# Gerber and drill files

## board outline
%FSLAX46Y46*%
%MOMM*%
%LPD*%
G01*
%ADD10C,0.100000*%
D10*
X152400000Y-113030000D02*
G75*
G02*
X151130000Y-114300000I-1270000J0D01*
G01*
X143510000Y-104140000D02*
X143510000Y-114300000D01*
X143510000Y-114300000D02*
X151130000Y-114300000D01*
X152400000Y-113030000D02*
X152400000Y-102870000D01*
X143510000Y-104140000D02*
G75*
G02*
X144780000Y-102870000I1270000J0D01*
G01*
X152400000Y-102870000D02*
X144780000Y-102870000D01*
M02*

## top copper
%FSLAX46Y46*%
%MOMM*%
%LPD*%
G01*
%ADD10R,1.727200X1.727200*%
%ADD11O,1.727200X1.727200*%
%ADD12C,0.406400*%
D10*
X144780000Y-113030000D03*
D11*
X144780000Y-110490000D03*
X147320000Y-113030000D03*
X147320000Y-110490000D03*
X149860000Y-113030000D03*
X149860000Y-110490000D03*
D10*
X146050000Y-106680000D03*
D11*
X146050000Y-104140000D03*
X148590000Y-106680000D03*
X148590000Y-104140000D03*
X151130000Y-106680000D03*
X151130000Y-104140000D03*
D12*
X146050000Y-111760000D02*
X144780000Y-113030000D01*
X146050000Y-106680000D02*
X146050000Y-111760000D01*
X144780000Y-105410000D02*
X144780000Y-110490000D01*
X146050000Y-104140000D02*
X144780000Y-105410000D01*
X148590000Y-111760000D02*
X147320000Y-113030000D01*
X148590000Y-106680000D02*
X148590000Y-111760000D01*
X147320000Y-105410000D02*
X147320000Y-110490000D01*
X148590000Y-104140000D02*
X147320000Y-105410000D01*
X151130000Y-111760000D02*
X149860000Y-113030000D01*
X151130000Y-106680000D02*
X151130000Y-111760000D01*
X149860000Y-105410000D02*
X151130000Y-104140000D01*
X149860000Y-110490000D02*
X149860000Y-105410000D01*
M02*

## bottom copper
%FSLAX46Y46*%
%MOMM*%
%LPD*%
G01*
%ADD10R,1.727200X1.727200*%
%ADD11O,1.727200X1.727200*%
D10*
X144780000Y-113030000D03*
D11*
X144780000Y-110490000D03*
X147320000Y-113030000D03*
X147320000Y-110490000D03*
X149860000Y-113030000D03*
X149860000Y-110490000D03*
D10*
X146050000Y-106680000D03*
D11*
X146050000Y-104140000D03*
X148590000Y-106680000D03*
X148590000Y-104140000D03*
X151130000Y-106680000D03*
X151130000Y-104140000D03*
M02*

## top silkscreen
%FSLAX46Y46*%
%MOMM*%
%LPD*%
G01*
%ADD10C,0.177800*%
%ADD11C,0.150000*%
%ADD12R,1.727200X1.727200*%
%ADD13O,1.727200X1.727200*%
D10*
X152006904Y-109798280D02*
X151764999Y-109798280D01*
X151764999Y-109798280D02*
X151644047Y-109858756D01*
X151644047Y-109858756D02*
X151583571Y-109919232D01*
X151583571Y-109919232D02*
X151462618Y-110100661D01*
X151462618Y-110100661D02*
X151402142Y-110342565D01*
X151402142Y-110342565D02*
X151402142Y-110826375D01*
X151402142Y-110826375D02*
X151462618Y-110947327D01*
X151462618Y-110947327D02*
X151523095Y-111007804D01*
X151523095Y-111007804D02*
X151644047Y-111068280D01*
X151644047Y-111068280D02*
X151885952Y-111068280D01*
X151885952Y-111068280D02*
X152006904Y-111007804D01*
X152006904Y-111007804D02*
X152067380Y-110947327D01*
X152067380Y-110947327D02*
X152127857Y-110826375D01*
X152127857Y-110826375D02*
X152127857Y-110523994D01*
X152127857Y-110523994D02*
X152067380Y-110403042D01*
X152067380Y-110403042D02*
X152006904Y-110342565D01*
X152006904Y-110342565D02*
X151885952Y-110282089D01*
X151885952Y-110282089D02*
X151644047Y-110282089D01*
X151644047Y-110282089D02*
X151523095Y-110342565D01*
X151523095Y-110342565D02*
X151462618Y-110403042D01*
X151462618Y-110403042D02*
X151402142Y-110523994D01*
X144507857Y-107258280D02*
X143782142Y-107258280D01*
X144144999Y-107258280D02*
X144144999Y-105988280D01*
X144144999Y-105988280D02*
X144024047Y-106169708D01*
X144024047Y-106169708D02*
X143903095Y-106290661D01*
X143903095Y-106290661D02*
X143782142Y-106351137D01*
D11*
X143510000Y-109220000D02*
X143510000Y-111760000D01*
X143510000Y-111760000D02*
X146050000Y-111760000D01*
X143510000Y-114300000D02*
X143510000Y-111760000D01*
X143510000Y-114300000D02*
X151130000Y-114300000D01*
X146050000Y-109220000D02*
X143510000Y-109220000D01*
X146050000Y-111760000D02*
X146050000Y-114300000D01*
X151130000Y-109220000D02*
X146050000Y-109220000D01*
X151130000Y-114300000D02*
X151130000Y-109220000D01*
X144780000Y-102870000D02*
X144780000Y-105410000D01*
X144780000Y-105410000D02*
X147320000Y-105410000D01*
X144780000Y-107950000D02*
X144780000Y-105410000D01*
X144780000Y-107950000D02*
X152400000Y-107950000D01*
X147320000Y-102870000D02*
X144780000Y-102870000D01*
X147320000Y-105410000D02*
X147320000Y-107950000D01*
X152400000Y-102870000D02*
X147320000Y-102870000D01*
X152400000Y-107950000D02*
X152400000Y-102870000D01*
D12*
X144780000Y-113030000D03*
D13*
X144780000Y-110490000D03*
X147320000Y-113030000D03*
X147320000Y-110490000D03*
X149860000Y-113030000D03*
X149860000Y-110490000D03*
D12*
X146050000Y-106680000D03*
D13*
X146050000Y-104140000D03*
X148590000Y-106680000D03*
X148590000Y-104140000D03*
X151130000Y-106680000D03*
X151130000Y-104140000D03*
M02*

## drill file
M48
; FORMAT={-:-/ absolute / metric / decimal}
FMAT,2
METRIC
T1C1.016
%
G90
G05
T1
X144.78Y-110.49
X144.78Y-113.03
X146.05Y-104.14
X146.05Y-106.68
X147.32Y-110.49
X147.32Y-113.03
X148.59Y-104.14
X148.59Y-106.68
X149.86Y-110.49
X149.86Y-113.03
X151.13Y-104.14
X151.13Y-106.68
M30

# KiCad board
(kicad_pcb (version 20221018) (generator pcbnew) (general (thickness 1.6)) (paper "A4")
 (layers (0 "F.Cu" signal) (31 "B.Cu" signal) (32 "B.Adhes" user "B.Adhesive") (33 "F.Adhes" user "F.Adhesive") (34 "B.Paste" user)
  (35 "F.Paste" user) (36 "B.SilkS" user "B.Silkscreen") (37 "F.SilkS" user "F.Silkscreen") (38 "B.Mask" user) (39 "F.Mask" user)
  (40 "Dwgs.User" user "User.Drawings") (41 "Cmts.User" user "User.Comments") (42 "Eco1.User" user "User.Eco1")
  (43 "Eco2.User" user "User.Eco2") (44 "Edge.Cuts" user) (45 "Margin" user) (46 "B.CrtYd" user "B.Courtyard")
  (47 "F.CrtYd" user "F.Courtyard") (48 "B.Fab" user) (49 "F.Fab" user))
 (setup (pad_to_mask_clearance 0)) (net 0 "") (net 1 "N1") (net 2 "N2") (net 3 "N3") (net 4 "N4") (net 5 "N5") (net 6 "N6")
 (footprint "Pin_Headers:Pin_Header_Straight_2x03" (layer "F.Cu") (at 147.32 111.76)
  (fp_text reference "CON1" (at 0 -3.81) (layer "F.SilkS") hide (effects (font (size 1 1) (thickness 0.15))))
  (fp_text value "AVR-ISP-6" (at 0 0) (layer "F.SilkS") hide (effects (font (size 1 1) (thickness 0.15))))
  (fp_line (start -3.81 -2.54) (end -3.81 0) (stroke (width 0.15) (type solid)) (layer "F.SilkS"))
  (fp_line (start -3.81 0) (end -1.27 0) (stroke (width 0.15) (type solid)) (layer "F.SilkS"))
  (fp_line (start -3.81 2.54) (end -3.81 0) (stroke (width 0.15) (type solid)) (layer "F.SilkS"))
  (fp_line (start -3.81 2.54) (end 3.81 2.54) (stroke (width 0.15) (type solid)) (layer "F.SilkS"))
  (fp_line (start -1.27 -2.54) (end -3.81 -2.54) (stroke (width 0.15) (type solid)) (layer "F.SilkS"))
  (fp_line (start -1.27 0) (end -1.27 2.54) (stroke (width 0.15) (type solid)) (layer "F.SilkS"))
  (fp_line (start 3.81 -2.54) (end -1.27 -2.54) (stroke (width 0.15) (type solid)) (layer "F.SilkS"))
  (fp_line (start 3.81 2.54) (end 3.81 -2.54) (stroke (width 0.15) (type solid)) (layer "F.SilkS"))
  (pad "1" thru_hole rect (at -2.54 1.27) (size 1.7272 1.7272) (drill 1.016) (layers "*.Cu" "*.Mask" "F.SilkS") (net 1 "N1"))
  (pad "2" thru_hole oval (at -2.54 -1.27) (size 1.7272 1.7272) (drill 1.016) (layers "*.Cu" "*.Mask" "F.SilkS") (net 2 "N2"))
  (pad "3" thru_hole oval (at 0 1.27) (size 1.7272 1.7272) (drill 1.016) (layers "*.Cu" "*.Mask" "F.SilkS") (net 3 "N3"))
  (pad "4" thru_hole oval (at 0 -1.27) (size 1.7272 1.7272) (drill 1.016) (layers "*.Cu" "*.Mask" "F.SilkS") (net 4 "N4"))
  (pad "5" thru_hole oval (at 2.54 1.27) (size 1.7272 1.7272) (drill 1.016) (layers "*.Cu" "*.Mask" "F.SilkS") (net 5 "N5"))
  (pad "6" thru_hole oval (at 2.54 -1.27) (size 1.7272 1.7272) (drill 1.016) (layers "*.Cu" "*.Mask" "F.SilkS") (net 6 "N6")))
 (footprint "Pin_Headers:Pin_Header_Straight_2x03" (layer "F.Cu") (at 148.59 105.41)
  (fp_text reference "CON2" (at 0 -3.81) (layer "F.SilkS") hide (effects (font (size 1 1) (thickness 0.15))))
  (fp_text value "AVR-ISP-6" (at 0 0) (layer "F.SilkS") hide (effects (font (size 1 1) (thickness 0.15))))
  (fp_line (start -3.81 -2.54) (end -3.81 0) (stroke (width 0.15) (type solid)) (layer "F.SilkS"))
  (fp_line (start -3.81 0) (end -1.27 0) (stroke (width 0.15) (type solid)) (layer "F.SilkS"))
  (fp_line (start -3.81 2.54) (end -3.81 0) (stroke (width 0.15) (type solid)) (layer "F.SilkS"))
  (fp_line (start -3.81 2.54) (end 3.81 2.54) (stroke (width 0.15) (type solid)) (layer "F.SilkS"))
  (fp_line (start -1.27 -2.54) (end -3.81 -2.54) (stroke (width 0.15) (type solid)) (layer "F.SilkS"))
  (fp_line (start -1.27 0) (end -1.27 2.54) (stroke (width 0.15) (type solid)) (layer "F.SilkS"))
  (fp_line (start 3.81 -2.54) (end -1.27 -2.54) (stroke (width 0.15) (type solid)) (layer "F.SilkS"))
  (fp_line (start 3.81 2.54) (end 3.81 -2.54) (stroke (width 0.15) (type solid)) (layer "F.SilkS"))
  (pad "1" thru_hole rect (at -2.54 1.27) (size 1.7272 1.7272) (drill 1.016) (layers "*.Cu" "*.Mask" "F.SilkS") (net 1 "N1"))
  (pad "2" thru_hole oval (at -2.54 -1.27) (size 1.7272 1.7272) (drill 1.016) (layers "*.Cu" "*.Mask" "F.SilkS") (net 2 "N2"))
  (pad "3" thru_hole oval (at 0 1.27) (size 1.7272 1.7272) (drill 1.016) (layers "*.Cu" "*.Mask" "F.SilkS") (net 3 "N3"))
  (pad "4" thru_hole oval (at 0 -1.27) (size 1.7272 1.7272) (drill 1.016) (layers "*.Cu" "*.Mask" "F.SilkS") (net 4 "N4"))
  (pad "5" thru_hole oval (at 2.54 1.27) (size 1.7272 1.7272) (drill 1.016) (layers "*.Cu" "*.Mask" "F.SilkS") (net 5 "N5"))
  (pad "6" thru_hole oval (at 2.54 -1.27) (size 1.7272 1.7272) (drill 1.016) (layers "*.Cu" "*.Mask" "F.SilkS") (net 6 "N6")))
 (gr_arc (start 152.4 113.03) (mid 152.028026 113.928026) (end 151.13 114.3) (stroke (width 0.1) (type solid)) (layer "Edge.Cuts"))
 (gr_line (start 143.51 104.14) (end 143.51 114.3) (stroke (width 0.1) (type solid)) (layer "Edge.Cuts"))
 (gr_line (start 143.51 114.3) (end 151.13 114.3) (stroke (width 0.1) (type solid)) (layer "Edge.Cuts"))
 (gr_line (start 152.4 113.03) (end 152.4 102.87) (stroke (width 0.1) (type solid)) (layer "Edge.Cuts"))
 (gr_arc (start 143.51 104.14) (mid 143.881974 103.241974) (end 144.78 102.87) (stroke (width 0.1) (type solid)) (layer "Edge.Cuts"))
 (gr_line (start 152.4 102.87) (end 144.78 102.87) (stroke (width 0.1) (type solid)) (layer "Edge.Cuts"))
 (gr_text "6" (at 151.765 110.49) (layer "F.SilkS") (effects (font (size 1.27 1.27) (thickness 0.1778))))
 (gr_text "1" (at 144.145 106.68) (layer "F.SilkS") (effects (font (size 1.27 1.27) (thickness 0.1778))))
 (segment (start 146.05 111.76) (end 144.78 113.03) (width 0.4064) (layer "F.Cu") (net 1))
 (segment (start 146.05 106.68) (end 146.05 111.76) (width 0.4064) (layer "F.Cu") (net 1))
 (segment (start 144.78 105.41) (end 144.78 110.49) (width 0.4064) (layer "F.Cu") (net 2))
 (segment (start 146.05 104.14) (end 144.78 105.41) (width 0.4064) (layer "F.Cu") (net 2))
 (segment (start 148.59 111.76) (end 147.32 113.03) (width 0.4064) (layer "F.Cu") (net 3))
 (segment (start 148.59 106.68) (end 148.59 111.76) (width 0.4064) (layer "F.Cu") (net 3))
 (segment (start 147.32 105.41) (end 147.32 110.49) (width 0.4064) (layer "F.Cu") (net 4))
 (segment (start 148.59 104.14) (end 147.32 105.41) (width 0.4064) (layer "F.Cu") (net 4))
 (segment (start 151.13 111.76) (end 149.86 113.03) (width 0.4064) (layer "F.Cu") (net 5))
 (segment (start 151.13 106.68) (end 151.13 111.76) (width 0.4064) (layer "F.Cu") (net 5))
 (segment (start 149.86 105.41) (end 151.13 104.14) (width 0.4064) (layer "F.Cu") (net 6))
 (segment (start 149.86 110.49) (end 149.86 105.41) (width 0.4064) (layer "F.Cu") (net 6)))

